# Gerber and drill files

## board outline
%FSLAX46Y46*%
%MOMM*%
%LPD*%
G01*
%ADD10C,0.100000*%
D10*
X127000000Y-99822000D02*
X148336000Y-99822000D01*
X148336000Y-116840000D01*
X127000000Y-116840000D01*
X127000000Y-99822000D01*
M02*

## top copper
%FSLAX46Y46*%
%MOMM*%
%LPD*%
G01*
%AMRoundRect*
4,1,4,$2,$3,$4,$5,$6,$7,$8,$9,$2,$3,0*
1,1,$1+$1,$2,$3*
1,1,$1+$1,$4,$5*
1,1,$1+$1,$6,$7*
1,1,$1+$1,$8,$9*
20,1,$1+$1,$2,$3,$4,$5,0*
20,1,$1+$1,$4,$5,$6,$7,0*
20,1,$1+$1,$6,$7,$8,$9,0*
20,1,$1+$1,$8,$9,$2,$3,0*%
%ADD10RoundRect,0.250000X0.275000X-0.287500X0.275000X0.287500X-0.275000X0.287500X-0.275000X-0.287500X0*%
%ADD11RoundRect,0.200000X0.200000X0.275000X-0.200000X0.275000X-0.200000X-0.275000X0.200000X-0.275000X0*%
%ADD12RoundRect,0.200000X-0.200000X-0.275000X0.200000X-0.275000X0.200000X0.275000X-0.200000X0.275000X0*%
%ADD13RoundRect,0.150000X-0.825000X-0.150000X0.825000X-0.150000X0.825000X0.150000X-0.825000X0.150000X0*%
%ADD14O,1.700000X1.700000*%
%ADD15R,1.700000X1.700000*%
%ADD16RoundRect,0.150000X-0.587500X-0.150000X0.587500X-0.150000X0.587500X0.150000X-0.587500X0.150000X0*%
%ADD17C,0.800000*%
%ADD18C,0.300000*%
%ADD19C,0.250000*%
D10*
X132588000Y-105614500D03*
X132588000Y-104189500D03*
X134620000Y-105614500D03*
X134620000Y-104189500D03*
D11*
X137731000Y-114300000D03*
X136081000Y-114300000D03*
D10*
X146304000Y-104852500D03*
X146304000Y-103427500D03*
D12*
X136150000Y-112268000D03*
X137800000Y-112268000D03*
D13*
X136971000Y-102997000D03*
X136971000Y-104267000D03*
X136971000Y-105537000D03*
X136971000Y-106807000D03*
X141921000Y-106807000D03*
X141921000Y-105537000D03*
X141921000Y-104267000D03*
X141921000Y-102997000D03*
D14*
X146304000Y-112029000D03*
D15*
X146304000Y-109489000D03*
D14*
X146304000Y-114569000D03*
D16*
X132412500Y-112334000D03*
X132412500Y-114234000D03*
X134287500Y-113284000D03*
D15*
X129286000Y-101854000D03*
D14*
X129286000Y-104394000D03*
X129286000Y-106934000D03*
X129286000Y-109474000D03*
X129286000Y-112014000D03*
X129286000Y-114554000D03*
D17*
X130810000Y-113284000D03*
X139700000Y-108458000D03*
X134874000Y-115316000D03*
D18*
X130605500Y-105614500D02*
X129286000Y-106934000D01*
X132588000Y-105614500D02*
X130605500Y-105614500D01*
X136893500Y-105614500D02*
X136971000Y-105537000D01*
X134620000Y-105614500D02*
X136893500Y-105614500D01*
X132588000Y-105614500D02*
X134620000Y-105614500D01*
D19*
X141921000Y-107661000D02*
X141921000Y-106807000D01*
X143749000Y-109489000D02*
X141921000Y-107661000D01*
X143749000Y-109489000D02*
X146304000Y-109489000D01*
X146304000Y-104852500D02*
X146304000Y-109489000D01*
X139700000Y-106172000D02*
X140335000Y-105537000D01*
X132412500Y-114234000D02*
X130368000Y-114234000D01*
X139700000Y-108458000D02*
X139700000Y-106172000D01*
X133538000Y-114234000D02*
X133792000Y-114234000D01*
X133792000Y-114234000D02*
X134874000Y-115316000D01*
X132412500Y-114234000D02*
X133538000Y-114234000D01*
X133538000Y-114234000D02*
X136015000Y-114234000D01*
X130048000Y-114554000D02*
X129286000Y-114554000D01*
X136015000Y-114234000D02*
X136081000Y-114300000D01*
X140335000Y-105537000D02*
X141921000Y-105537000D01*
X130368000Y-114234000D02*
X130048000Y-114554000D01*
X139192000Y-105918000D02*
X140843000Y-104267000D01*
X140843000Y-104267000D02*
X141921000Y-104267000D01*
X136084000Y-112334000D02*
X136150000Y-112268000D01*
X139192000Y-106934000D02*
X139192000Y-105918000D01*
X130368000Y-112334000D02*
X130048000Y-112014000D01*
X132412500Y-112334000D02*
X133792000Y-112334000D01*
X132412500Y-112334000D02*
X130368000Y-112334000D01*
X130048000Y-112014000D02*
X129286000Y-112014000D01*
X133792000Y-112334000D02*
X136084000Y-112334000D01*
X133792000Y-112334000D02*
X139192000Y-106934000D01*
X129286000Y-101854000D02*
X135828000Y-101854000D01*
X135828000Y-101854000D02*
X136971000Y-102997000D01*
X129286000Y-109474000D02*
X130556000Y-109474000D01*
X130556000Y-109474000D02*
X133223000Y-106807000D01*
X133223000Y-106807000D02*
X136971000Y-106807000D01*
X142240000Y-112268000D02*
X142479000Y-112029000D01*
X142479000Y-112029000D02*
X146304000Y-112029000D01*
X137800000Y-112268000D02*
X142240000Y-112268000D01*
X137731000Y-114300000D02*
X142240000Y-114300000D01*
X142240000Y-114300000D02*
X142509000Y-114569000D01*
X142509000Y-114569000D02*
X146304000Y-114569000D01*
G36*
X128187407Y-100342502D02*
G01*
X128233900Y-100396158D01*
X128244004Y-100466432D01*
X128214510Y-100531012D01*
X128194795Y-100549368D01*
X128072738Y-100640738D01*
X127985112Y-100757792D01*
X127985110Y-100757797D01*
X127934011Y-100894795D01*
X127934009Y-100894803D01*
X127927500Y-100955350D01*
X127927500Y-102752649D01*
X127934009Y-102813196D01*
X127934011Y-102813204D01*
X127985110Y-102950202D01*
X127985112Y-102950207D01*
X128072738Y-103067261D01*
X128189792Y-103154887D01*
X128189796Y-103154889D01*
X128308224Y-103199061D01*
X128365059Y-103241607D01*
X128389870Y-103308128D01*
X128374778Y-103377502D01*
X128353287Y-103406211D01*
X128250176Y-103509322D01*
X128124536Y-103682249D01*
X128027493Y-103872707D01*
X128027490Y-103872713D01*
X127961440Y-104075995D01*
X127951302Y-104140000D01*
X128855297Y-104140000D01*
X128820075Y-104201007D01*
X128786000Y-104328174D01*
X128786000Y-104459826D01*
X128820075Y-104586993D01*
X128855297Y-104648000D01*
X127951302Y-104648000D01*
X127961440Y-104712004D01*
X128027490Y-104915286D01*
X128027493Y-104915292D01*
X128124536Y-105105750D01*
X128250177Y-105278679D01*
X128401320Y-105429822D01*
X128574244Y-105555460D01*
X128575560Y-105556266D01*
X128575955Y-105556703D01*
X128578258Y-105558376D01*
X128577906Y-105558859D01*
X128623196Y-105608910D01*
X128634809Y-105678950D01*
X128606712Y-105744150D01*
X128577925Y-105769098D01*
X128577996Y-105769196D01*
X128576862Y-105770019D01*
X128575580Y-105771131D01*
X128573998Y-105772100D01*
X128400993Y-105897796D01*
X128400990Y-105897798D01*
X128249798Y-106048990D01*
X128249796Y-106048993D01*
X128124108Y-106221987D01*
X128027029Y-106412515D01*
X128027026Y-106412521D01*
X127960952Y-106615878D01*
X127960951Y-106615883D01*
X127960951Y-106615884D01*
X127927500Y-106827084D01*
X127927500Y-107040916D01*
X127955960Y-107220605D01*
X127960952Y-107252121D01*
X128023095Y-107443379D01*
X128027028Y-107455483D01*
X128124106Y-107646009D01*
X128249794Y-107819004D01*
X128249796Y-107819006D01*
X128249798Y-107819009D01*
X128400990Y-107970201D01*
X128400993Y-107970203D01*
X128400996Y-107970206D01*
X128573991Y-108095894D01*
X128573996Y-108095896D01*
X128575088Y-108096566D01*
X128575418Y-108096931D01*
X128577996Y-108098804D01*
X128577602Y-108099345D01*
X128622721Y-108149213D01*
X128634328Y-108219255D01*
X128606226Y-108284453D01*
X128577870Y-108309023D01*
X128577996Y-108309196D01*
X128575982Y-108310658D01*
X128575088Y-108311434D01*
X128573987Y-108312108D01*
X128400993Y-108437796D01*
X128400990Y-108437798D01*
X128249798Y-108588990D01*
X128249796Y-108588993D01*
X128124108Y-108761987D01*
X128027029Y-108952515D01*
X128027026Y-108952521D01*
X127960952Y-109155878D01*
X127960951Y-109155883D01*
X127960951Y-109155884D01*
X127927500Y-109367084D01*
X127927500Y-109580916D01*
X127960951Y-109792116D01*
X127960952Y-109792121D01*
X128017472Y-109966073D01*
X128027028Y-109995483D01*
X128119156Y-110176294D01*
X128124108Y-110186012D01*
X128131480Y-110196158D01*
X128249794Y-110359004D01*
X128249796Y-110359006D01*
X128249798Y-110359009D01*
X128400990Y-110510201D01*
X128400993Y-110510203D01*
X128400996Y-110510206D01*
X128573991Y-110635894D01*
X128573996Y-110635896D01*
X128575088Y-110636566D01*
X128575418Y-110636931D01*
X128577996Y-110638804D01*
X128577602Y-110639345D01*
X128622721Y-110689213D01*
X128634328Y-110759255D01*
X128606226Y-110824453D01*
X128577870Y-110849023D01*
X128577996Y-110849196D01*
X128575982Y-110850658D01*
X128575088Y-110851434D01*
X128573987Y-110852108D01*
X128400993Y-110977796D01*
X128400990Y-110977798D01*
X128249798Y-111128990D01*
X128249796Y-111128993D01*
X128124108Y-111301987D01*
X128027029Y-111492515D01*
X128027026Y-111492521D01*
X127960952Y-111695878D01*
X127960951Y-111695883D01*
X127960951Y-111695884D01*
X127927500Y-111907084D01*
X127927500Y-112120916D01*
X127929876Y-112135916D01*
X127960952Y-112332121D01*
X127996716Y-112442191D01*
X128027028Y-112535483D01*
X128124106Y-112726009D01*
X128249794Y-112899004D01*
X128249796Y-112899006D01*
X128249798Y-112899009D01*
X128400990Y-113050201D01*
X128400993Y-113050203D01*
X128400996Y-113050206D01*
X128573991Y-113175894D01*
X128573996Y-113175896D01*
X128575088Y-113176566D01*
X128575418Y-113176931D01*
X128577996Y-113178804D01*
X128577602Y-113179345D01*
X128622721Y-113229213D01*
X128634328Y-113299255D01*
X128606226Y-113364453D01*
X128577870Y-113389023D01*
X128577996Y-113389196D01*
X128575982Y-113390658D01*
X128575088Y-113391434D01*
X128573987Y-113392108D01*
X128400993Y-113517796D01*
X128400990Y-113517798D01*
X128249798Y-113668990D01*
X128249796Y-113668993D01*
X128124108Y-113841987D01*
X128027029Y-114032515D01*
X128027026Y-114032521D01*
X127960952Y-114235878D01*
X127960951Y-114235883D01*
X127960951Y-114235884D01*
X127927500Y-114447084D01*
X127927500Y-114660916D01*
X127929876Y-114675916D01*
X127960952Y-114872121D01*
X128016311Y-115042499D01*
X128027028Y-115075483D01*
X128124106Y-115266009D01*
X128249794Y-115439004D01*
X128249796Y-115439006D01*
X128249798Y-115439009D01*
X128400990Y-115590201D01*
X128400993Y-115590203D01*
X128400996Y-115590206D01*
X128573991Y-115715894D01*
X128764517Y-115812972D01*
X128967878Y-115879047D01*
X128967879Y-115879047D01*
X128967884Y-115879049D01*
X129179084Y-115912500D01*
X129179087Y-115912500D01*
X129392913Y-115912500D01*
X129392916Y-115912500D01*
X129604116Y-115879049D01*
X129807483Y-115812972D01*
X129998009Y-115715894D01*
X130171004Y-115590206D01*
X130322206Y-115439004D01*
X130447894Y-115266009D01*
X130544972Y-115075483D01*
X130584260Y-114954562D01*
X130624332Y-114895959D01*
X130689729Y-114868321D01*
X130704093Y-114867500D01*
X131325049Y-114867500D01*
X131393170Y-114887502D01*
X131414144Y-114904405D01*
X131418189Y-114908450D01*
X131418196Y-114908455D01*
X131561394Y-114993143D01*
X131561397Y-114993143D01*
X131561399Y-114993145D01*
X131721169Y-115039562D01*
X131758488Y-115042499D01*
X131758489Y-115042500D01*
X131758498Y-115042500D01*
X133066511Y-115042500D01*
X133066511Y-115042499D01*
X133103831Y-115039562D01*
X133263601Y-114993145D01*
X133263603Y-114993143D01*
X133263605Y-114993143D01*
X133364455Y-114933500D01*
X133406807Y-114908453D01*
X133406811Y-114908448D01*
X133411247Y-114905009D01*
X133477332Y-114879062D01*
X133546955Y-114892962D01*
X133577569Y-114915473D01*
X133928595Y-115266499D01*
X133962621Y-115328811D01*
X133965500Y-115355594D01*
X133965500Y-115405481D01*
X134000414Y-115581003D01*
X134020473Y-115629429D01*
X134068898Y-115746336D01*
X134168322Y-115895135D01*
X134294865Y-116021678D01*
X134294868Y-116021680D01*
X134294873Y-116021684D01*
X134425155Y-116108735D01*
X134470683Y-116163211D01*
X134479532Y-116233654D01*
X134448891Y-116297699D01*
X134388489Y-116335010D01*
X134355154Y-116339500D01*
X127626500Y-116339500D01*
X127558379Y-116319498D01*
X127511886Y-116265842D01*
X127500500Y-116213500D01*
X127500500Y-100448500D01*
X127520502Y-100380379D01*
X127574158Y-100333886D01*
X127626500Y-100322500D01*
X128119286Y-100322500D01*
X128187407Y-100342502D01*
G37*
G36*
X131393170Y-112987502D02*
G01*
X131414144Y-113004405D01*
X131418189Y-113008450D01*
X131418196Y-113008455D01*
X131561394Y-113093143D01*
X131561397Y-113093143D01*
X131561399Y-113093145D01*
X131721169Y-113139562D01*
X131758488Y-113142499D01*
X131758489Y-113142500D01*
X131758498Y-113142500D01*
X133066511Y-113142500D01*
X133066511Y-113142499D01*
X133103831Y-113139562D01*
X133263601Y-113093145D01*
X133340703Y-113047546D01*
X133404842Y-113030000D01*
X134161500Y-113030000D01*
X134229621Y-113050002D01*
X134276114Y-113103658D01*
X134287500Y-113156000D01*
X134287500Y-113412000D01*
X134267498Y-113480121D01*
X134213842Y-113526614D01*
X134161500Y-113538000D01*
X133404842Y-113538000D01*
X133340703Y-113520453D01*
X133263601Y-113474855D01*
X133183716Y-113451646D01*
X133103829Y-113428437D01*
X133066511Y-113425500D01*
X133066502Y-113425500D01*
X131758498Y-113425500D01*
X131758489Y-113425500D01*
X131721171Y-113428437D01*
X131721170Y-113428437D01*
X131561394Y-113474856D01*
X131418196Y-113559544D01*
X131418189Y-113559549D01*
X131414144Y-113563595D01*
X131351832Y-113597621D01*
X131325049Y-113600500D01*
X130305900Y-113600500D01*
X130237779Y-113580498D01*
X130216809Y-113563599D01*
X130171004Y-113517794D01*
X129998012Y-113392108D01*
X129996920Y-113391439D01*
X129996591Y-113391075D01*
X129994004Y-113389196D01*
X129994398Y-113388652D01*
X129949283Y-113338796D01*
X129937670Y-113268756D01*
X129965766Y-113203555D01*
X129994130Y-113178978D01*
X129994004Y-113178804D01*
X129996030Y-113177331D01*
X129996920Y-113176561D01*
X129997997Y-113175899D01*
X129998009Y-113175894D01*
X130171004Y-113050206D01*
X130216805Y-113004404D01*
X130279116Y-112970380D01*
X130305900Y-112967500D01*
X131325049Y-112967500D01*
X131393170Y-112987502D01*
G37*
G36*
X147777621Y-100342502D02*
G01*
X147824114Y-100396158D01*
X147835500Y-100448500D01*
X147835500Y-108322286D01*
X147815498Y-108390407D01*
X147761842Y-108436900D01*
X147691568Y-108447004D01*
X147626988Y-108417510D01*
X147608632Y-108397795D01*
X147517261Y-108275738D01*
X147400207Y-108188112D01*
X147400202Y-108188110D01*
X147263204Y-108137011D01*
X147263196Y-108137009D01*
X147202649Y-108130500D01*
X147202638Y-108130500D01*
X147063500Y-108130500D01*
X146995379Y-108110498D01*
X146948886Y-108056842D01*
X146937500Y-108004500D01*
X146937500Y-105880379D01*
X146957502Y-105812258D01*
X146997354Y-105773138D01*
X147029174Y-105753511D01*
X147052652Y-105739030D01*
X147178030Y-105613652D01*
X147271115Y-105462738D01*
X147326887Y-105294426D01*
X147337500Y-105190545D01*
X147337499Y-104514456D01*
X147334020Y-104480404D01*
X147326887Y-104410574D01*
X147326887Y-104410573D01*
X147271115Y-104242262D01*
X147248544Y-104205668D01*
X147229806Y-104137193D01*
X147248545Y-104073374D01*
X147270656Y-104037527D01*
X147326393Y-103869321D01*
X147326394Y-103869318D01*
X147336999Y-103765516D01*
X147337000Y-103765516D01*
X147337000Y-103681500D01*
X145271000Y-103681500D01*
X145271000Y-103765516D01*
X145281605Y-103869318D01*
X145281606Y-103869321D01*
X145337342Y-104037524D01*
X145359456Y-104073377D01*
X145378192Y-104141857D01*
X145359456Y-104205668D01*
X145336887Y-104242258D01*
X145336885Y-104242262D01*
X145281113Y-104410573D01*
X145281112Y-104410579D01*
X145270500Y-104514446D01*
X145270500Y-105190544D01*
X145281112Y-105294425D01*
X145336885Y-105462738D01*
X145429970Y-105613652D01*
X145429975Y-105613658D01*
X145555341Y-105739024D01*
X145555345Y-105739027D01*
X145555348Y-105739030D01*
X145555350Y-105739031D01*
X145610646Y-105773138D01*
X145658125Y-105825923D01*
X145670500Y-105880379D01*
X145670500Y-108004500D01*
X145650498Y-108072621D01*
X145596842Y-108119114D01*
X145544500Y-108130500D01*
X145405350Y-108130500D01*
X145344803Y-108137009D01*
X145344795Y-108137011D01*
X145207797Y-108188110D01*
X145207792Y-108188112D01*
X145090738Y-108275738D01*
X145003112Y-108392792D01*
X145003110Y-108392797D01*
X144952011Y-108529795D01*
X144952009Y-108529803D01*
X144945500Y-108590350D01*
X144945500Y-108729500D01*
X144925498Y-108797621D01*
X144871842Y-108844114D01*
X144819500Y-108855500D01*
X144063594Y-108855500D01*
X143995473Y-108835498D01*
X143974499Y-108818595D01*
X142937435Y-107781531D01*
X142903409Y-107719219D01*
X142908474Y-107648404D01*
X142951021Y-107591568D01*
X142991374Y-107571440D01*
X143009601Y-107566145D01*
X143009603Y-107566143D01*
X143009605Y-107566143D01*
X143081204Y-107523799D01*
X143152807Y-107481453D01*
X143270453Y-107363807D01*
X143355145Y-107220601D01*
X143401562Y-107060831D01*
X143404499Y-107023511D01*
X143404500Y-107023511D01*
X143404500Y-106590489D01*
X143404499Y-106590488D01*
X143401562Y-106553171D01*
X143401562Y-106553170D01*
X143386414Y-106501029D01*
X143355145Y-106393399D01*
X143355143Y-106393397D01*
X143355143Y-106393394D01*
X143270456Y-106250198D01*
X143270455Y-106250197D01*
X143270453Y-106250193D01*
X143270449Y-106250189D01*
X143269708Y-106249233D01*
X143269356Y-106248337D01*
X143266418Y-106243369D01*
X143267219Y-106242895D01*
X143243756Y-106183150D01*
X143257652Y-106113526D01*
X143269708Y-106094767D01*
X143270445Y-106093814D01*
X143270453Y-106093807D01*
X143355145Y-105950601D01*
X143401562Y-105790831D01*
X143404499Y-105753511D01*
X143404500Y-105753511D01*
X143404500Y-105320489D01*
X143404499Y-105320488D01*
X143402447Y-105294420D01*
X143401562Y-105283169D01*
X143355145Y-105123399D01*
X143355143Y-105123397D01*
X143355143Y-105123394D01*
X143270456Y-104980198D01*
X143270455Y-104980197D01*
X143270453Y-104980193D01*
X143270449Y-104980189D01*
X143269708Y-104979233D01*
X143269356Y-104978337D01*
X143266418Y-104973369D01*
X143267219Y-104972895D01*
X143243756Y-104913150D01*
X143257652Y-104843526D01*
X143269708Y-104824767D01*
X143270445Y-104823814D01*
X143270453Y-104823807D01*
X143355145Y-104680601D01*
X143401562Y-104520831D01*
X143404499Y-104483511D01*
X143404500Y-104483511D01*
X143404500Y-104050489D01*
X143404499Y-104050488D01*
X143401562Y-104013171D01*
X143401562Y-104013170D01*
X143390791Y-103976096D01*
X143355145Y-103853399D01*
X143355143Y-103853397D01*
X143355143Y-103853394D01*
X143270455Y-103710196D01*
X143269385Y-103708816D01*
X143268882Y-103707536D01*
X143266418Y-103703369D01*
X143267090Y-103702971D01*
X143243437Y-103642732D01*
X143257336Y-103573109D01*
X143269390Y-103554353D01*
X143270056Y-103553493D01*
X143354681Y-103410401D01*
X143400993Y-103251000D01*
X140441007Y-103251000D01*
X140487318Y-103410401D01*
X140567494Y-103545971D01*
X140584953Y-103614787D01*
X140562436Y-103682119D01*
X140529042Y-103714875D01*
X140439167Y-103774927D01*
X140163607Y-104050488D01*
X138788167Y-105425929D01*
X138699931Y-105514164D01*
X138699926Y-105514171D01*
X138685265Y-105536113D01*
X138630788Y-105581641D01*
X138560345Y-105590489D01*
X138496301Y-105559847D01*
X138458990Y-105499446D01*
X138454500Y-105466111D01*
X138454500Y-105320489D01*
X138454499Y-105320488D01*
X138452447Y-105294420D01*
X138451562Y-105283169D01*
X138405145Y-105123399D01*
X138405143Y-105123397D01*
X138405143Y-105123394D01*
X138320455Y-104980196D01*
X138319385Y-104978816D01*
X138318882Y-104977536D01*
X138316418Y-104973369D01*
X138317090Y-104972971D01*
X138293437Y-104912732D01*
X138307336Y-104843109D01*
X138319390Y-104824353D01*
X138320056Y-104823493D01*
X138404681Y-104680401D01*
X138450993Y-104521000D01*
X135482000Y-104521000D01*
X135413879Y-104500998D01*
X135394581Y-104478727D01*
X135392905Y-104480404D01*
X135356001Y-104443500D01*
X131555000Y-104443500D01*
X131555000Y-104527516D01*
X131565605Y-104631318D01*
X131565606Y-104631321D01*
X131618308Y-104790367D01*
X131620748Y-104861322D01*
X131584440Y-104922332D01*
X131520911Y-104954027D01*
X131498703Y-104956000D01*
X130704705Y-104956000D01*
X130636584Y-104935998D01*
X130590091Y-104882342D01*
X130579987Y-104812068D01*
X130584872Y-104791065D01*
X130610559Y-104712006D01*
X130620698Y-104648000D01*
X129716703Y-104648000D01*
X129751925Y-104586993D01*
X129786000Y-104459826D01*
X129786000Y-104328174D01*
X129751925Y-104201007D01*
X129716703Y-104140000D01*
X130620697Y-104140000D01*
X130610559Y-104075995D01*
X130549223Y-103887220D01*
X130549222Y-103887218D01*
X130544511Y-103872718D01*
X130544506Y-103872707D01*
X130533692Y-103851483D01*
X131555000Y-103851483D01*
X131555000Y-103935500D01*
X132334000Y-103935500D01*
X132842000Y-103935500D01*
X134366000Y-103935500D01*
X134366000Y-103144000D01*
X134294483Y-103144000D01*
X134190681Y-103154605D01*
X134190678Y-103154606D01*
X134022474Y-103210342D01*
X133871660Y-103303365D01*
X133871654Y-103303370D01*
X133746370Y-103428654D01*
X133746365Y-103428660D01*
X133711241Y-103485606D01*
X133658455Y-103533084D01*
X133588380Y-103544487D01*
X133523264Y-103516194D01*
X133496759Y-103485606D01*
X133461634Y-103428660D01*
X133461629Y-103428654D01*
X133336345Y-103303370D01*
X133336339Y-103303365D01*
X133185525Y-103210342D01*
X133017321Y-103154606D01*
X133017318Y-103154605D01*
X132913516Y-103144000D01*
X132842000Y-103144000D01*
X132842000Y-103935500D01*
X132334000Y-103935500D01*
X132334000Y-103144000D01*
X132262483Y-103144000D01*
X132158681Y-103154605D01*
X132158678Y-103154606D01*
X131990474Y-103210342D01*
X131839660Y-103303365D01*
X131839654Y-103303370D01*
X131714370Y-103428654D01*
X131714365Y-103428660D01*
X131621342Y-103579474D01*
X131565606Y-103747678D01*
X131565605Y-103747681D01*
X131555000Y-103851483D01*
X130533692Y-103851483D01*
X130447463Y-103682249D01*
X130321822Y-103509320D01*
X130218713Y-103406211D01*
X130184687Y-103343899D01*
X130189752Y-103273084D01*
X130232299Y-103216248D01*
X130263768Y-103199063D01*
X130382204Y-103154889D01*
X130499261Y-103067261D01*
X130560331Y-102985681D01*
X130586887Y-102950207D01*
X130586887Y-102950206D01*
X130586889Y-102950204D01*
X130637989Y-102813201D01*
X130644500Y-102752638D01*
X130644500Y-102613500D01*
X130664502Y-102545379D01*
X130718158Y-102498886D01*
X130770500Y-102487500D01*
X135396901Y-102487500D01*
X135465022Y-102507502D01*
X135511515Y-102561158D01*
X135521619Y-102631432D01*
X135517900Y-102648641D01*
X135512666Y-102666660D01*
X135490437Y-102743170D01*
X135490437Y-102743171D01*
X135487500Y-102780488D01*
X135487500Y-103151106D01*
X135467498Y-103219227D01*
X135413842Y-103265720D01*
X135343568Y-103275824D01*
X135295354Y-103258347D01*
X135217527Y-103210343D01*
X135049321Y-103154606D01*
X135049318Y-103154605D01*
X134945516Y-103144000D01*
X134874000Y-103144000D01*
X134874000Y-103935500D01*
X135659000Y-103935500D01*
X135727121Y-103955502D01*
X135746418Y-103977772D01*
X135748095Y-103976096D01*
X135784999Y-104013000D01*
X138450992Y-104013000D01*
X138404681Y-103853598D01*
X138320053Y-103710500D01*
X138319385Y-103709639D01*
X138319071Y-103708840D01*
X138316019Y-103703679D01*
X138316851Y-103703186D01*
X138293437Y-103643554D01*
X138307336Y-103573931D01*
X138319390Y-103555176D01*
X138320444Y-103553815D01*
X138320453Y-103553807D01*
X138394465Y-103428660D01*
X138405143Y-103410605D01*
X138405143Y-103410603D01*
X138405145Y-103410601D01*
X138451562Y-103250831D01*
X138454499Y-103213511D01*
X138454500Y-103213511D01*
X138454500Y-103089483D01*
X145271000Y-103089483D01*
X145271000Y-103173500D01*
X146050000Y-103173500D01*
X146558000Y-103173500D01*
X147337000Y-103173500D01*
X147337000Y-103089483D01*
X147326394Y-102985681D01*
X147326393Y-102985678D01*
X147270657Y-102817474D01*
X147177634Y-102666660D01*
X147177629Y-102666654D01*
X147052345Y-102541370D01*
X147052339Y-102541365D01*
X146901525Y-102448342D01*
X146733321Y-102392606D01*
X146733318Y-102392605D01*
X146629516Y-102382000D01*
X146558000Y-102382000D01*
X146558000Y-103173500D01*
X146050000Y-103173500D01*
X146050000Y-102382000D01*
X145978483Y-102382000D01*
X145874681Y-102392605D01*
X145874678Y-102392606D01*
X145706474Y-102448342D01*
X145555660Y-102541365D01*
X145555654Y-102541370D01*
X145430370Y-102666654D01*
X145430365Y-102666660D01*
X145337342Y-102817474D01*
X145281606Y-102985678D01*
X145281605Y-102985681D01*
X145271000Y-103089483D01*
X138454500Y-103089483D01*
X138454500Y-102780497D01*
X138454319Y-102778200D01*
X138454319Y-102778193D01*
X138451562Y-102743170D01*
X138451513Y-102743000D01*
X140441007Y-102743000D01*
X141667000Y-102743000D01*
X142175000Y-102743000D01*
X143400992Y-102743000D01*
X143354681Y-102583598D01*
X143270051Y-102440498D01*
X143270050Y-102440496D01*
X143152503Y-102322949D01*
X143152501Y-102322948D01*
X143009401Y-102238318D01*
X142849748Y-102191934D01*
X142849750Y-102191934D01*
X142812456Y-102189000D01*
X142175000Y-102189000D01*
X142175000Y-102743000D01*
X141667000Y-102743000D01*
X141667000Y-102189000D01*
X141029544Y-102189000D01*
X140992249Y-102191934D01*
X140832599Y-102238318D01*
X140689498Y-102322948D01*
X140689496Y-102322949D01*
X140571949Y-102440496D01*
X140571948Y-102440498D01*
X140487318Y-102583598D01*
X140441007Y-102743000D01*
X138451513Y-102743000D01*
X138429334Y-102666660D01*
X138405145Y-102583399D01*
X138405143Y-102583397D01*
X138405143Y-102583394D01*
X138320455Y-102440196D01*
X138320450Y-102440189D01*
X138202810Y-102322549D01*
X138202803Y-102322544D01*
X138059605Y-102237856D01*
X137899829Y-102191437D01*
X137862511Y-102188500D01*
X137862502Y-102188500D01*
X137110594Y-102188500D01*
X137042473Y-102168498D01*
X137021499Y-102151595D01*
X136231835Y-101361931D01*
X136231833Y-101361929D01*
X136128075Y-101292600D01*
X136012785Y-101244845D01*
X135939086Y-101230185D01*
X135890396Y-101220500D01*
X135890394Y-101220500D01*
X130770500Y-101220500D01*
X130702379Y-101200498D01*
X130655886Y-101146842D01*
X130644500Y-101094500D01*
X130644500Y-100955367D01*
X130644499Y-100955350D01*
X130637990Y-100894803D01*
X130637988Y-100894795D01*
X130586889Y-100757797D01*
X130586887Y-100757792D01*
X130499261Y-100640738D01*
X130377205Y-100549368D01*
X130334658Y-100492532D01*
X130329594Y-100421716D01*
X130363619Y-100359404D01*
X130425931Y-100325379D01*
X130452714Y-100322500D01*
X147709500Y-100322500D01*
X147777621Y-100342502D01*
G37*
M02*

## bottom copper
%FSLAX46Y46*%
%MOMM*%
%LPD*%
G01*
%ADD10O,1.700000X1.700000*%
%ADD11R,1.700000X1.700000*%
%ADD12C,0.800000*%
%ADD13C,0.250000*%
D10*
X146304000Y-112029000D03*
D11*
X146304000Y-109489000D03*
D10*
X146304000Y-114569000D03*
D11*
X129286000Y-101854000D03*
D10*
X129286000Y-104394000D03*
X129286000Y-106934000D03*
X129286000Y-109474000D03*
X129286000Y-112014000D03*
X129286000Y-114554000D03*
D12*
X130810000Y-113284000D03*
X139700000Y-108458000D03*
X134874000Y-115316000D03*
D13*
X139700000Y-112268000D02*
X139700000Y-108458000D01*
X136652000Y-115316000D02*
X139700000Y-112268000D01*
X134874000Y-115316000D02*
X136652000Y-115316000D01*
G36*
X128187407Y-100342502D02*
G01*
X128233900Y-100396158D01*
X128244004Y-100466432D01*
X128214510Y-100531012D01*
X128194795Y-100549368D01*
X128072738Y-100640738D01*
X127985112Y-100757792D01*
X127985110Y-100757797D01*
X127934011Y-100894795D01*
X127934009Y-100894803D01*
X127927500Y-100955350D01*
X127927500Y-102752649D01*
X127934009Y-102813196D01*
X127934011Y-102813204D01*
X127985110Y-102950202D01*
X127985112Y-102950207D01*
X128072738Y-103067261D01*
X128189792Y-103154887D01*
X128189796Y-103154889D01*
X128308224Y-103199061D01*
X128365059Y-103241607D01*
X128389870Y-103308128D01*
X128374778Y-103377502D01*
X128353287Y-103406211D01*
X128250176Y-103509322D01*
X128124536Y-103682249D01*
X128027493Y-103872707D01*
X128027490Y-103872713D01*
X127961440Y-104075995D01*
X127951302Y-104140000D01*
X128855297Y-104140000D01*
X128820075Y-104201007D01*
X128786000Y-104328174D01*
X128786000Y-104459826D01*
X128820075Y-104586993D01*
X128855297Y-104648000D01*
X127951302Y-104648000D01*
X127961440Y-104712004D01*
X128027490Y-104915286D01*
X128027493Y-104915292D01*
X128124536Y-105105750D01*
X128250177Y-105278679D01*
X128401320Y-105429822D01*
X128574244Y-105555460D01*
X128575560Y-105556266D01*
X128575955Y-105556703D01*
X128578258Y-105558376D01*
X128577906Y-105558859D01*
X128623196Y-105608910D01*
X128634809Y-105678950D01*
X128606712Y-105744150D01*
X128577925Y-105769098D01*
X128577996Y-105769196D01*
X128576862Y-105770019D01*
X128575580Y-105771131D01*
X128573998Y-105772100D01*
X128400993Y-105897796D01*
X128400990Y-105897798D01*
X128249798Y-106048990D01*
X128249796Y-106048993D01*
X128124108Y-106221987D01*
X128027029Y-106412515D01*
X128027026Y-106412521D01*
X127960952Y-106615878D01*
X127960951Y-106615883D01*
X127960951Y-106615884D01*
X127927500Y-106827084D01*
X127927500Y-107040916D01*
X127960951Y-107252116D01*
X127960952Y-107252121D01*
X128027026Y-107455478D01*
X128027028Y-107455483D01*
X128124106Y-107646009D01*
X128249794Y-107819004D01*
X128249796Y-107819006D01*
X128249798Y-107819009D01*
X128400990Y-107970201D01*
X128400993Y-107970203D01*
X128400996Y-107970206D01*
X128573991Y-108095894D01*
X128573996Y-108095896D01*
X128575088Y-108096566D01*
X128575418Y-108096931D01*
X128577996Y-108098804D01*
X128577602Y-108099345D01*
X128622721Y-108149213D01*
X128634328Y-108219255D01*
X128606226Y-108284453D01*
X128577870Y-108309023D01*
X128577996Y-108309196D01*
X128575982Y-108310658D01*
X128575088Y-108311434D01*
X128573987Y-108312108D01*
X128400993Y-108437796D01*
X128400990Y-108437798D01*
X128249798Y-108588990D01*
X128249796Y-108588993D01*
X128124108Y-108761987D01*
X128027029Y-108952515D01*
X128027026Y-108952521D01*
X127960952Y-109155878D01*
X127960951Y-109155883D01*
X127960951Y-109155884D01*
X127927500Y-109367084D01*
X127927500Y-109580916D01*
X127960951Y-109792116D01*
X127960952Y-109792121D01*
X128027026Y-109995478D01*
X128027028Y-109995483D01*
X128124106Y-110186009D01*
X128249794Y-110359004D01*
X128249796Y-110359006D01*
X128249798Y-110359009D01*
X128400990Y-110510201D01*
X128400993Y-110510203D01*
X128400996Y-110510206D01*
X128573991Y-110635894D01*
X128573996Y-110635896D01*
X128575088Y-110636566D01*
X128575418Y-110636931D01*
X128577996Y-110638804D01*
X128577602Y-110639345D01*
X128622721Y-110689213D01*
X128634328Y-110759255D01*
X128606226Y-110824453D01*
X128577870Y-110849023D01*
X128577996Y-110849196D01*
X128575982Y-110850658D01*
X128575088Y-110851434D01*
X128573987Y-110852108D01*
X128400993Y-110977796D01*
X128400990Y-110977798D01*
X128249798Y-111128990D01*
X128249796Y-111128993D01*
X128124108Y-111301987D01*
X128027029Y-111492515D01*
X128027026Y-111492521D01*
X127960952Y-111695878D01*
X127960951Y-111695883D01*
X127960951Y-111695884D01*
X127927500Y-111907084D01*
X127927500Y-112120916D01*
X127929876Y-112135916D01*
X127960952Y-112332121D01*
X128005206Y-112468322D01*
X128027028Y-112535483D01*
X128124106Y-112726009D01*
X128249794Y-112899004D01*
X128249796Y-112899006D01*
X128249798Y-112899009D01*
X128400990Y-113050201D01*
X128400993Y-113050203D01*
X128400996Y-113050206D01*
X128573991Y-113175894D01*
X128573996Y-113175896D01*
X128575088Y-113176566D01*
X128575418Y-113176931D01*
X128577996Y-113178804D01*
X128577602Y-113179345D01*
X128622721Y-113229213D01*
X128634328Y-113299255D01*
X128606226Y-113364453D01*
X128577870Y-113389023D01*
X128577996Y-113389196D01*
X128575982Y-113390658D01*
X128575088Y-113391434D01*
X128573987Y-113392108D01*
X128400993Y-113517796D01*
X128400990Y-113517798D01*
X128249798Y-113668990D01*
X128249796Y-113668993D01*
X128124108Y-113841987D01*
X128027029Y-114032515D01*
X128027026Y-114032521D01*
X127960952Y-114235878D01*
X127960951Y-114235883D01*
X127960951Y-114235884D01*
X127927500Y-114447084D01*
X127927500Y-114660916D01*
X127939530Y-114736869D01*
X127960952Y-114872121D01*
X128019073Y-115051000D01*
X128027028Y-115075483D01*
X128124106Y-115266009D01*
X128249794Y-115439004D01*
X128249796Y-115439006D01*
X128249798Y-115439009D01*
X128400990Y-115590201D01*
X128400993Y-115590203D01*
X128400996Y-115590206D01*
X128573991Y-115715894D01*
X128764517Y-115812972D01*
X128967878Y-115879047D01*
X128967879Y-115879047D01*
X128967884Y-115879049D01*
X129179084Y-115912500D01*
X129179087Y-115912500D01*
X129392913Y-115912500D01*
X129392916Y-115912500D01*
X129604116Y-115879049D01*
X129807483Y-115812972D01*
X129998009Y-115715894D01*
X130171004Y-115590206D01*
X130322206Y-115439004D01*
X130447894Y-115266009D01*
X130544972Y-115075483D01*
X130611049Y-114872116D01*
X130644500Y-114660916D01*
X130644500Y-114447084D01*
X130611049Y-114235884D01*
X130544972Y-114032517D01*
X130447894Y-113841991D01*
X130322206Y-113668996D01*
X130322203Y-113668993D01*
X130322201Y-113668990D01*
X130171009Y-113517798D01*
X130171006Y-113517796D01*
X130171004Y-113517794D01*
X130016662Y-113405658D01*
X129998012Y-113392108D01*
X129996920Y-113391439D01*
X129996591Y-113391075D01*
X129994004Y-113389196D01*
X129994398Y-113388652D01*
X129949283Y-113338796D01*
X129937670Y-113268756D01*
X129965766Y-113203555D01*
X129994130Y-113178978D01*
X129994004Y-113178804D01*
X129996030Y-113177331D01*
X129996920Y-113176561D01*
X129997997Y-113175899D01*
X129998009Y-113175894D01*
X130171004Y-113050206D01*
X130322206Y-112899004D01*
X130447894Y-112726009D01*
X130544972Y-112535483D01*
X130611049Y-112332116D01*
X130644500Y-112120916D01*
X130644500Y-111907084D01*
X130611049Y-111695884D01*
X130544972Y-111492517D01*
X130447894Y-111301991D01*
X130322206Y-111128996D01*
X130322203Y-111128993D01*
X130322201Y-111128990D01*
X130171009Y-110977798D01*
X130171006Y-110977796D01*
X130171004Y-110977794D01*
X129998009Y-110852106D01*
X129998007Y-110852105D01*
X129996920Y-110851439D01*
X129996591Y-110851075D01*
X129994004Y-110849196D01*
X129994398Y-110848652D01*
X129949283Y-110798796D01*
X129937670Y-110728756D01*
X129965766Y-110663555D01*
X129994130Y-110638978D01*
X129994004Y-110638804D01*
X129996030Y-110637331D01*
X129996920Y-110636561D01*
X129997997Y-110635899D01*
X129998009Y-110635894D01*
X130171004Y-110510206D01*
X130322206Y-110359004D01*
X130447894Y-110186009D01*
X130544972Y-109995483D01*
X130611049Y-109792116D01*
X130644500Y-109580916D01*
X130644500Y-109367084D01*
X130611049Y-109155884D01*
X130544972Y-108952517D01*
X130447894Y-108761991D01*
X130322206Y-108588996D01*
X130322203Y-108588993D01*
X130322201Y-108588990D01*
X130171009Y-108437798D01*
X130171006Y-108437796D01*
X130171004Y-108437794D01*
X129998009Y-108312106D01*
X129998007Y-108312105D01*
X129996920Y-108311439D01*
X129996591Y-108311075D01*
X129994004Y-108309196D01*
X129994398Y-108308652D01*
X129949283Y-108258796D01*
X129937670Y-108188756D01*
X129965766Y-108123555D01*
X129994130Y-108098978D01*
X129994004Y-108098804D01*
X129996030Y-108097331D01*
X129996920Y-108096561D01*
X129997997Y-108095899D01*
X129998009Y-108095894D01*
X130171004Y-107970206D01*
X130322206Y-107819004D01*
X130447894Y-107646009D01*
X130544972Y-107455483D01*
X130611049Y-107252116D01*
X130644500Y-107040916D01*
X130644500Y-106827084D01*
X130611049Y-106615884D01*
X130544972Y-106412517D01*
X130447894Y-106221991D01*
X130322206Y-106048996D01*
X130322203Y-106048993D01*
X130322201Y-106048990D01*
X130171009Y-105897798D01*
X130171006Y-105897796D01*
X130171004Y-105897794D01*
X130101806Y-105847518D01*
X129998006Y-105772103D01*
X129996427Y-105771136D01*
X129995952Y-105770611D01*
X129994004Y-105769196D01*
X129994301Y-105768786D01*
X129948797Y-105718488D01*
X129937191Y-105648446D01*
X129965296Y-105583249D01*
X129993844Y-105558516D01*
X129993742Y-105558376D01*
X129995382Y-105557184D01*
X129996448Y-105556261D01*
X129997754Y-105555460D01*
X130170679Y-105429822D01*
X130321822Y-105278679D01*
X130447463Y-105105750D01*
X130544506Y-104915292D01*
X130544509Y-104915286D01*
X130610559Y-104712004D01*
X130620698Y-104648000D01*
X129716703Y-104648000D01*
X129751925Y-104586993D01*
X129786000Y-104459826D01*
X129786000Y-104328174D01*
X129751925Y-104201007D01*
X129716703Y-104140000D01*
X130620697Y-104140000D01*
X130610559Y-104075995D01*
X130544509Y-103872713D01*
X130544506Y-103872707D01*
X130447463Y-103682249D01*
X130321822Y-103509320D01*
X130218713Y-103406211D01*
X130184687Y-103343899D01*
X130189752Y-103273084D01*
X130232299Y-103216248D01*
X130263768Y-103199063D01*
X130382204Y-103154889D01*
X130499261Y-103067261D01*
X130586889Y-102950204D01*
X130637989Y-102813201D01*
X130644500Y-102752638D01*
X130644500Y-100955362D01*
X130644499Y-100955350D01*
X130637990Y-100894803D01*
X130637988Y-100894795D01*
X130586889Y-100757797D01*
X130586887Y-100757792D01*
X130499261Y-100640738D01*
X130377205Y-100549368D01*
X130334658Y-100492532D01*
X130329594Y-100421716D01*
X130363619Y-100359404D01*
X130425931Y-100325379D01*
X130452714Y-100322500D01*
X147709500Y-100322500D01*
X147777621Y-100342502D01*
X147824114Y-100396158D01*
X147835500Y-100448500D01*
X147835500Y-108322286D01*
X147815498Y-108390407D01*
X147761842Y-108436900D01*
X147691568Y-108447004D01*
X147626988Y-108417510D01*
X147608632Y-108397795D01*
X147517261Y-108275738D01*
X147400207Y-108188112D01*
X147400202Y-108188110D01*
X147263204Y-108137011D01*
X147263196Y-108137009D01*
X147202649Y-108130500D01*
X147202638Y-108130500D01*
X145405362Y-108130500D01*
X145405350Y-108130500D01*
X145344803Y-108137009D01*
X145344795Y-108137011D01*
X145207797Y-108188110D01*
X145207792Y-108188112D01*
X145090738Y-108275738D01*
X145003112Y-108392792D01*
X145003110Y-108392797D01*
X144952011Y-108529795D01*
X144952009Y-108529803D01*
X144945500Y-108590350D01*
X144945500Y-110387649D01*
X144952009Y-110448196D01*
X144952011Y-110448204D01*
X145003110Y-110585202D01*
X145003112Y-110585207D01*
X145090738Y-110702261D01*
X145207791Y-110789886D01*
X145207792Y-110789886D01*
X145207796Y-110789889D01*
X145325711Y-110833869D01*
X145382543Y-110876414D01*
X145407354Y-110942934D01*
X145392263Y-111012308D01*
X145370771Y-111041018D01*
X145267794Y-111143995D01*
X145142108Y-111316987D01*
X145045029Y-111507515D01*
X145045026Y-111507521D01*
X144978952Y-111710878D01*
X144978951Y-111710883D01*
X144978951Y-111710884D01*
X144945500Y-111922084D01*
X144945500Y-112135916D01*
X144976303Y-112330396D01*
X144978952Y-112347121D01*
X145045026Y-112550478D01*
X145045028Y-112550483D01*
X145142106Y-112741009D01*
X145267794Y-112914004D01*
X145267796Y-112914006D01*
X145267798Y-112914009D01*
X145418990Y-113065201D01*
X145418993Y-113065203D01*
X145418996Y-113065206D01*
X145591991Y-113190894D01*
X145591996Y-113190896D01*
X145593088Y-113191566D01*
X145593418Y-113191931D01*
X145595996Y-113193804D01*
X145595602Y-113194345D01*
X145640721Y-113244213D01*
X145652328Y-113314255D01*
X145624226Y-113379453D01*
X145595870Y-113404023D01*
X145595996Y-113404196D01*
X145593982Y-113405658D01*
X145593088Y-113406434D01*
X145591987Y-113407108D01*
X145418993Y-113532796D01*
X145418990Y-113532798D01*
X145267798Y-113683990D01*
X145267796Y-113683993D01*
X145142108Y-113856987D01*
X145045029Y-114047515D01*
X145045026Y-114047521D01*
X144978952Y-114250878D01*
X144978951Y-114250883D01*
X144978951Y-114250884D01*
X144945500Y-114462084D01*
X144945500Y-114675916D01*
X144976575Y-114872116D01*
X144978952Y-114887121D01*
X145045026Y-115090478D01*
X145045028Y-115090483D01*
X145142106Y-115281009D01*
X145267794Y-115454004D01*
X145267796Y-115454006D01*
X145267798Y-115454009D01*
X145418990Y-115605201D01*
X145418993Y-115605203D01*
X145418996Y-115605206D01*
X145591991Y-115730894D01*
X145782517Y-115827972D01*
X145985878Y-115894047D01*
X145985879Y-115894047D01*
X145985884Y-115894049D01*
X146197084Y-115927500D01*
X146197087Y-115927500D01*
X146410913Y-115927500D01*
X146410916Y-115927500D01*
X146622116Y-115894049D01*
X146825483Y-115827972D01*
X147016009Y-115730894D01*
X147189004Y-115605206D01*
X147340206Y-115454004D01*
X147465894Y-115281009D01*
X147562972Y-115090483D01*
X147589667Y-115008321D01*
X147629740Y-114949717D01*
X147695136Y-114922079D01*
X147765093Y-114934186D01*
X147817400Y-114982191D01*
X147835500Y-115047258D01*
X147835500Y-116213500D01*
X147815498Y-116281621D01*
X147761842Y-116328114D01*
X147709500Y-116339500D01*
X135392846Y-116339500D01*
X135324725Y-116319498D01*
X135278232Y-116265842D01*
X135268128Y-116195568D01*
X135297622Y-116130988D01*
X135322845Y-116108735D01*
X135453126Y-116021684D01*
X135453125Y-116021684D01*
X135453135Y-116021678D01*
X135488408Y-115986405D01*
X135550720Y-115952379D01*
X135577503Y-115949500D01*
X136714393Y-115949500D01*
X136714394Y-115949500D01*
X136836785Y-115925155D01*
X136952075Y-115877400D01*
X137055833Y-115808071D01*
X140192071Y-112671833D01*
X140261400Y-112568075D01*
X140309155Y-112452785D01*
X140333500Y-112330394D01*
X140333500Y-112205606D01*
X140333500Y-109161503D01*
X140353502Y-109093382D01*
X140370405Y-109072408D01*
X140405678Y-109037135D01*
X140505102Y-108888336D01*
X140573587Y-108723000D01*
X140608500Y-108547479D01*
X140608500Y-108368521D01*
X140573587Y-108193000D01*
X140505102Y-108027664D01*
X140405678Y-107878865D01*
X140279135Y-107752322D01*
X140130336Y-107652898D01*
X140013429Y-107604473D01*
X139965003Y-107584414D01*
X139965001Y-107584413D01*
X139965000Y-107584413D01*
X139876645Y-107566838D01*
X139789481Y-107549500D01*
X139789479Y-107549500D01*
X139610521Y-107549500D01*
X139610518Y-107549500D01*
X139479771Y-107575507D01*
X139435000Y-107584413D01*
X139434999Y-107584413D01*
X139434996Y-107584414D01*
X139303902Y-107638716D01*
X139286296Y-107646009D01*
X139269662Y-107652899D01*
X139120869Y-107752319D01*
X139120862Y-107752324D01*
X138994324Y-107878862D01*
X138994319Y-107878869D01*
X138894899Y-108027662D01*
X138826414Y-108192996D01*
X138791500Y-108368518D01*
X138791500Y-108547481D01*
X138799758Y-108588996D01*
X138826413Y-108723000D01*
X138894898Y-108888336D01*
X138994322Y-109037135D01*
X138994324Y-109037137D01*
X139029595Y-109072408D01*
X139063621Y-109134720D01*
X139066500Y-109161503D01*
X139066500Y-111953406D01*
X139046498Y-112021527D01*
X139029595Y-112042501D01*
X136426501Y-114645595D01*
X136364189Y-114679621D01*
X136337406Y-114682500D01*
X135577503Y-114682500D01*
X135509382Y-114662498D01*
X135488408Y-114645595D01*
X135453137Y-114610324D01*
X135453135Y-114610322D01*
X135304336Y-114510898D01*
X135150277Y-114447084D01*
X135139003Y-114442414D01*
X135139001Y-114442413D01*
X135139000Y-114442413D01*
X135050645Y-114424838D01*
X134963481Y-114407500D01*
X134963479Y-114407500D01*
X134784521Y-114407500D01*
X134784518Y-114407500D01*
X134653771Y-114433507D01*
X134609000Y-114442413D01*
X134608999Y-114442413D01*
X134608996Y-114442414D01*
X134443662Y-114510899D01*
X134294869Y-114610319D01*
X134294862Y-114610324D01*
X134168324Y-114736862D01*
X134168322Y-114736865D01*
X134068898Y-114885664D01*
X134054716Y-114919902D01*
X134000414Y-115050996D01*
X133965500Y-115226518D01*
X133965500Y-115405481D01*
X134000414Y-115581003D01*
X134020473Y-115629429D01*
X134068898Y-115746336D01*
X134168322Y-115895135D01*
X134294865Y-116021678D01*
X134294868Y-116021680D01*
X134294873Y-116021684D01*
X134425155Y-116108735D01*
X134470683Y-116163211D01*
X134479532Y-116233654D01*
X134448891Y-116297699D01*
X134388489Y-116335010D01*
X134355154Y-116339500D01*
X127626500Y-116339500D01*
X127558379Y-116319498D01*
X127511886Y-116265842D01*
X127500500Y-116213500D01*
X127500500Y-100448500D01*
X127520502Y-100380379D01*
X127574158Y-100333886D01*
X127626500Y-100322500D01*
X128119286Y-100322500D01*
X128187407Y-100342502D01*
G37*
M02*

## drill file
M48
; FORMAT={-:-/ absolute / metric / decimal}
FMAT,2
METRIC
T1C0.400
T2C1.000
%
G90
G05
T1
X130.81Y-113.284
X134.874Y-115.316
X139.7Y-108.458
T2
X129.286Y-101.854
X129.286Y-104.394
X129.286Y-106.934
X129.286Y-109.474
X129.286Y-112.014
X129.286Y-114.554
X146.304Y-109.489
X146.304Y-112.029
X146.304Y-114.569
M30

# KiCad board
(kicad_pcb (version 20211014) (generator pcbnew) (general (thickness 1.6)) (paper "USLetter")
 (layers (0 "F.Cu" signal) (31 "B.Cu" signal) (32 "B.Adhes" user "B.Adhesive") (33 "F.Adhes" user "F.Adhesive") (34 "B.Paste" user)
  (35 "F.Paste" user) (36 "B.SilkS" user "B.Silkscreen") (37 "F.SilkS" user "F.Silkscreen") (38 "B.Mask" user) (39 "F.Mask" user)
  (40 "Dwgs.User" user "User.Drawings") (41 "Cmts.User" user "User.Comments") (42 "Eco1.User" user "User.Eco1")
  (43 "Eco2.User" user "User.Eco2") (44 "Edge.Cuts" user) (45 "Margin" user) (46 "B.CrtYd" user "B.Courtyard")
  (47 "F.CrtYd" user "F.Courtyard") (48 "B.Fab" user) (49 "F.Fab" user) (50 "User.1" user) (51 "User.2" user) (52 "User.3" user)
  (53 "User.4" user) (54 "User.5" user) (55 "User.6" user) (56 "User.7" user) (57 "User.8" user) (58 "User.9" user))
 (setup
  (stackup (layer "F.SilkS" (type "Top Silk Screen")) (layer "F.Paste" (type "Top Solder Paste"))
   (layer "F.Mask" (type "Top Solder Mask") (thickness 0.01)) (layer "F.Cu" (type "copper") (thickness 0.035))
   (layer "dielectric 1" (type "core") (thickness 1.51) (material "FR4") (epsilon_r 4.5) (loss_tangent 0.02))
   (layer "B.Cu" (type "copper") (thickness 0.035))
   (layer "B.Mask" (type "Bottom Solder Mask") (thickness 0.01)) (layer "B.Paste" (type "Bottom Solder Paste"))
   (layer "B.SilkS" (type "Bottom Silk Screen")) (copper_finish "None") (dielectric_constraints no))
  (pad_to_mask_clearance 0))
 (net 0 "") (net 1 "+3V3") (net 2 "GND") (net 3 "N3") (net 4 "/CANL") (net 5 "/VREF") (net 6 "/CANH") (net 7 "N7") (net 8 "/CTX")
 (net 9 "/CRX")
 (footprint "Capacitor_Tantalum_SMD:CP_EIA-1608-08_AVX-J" (layer "F.Cu") (at 132.588 104.902 90)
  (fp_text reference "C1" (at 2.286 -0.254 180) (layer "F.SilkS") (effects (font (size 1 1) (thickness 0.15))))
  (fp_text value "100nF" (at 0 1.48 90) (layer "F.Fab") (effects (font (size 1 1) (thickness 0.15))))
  (pad "1" smd roundrect (at -0.7125 0 90) (size 1.075 1.05) (layers "F.Cu" "F.Paste" "F.Mask") (roundrect_rratio 0.238095) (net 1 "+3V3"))
  (pad "2" smd roundrect (at 0.7125 0 90) (size 1.075 1.05) (layers "F.Cu" "F.Paste" "F.Mask") (roundrect_rratio 0.238095) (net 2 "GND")))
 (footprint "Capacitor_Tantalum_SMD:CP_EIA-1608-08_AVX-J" (layer "F.Cu") (at 134.62 104.902 90)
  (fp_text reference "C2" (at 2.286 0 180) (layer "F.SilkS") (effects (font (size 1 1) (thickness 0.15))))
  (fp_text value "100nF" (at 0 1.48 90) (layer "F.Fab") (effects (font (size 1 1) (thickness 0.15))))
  (pad "1" smd roundrect (at -0.7125 0 90) (size 1.075 1.05) (layers "F.Cu" "F.Paste" "F.Mask") (roundrect_rratio 0.238095) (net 1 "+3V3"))
  (pad "2" smd roundrect (at 0.7125 0 90) (size 1.075 1.05) (layers "F.Cu" "F.Paste" "F.Mask") (roundrect_rratio 0.238095) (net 2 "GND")))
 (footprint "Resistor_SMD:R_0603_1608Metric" (layer "F.Cu") (at 136.906 114.3 180)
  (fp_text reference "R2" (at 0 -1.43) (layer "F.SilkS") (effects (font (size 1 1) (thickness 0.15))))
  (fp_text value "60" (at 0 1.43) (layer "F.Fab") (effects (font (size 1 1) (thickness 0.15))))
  (pad "1" smd roundrect (at -0.825 0 180) (size 0.8 0.95) (layers "F.Cu" "F.Paste" "F.Mask") (roundrect_rratio 0.25) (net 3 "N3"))
  (pad "2" smd roundrect (at 0.825 0 180) (size 0.8 0.95) (layers "F.Cu" "F.Paste" "F.Mask") (roundrect_rratio 0.25) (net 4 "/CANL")))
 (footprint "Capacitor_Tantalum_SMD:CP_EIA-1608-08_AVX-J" (layer "F.Cu") (at 146.304 104.14 90)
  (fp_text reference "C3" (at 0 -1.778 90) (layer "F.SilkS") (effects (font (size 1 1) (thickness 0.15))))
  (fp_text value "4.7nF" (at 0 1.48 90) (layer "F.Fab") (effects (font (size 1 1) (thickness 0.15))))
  (pad "1" smd roundrect (at -0.7125 0 90) (size 1.075 1.05) (layers "F.Cu" "F.Paste" "F.Mask") (roundrect_rratio 0.238095) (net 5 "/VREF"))
  (pad "2" smd roundrect (at 0.7125 0 90) (size 1.075 1.05) (layers "F.Cu" "F.Paste" "F.Mask") (roundrect_rratio 0.238095) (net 2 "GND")))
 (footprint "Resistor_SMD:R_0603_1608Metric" (layer "F.Cu") (at 136.975 112.268)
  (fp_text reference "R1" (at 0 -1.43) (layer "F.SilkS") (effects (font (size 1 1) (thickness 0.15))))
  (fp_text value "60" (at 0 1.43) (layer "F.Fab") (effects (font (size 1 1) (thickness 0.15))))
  (pad "1" smd roundrect (at -0.825 0) (size 0.8 0.95) (layers "F.Cu" "F.Paste" "F.Mask") (roundrect_rratio 0.25) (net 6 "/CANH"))
  (pad "2" smd roundrect (at 0.825 0) (size 0.8 0.95) (layers "F.Cu" "F.Paste" "F.Mask") (roundrect_rratio 0.25) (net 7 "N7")))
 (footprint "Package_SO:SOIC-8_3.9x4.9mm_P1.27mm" (layer "F.Cu") (at 139.446 104.902)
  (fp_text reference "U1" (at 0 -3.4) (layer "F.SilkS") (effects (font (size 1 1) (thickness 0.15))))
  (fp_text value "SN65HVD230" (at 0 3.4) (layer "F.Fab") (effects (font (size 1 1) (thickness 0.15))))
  (pad "1" smd roundrect (at -2.475 -1.905) (size 1.95 0.6) (layers "F.Cu" "F.Paste" "F.Mask") (roundrect_rratio 0.25) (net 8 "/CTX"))
  (pad "2" smd roundrect (at -2.475 -0.635) (size 1.95 0.6) (layers "F.Cu" "F.Paste" "F.Mask") (roundrect_rratio 0.25) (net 2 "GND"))
  (pad "3" smd roundrect (at -2.475 0.635) (size 1.95 0.6) (layers "F.Cu" "F.Paste" "F.Mask") (roundrect_rratio 0.25) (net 1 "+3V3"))
  (pad "4" smd roundrect (at -2.475 1.905) (size 1.95 0.6) (layers "F.Cu" "F.Paste" "F.Mask") (roundrect_rratio 0.25) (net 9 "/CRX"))
  (pad "5" smd roundrect (at 2.475 1.905) (size 1.95 0.6) (layers "F.Cu" "F.Paste" "F.Mask") (roundrect_rratio 0.25) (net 5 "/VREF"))
  (pad "6" smd roundrect (at 2.475 0.635) (size 1.95 0.6) (layers "F.Cu" "F.Paste" "F.Mask") (roundrect_rratio 0.25) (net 4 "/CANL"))
  (pad "7" smd roundrect (at 2.475 -0.635) (size 1.95 0.6) (layers "F.Cu" "F.Paste" "F.Mask") (roundrect_rratio 0.25) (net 6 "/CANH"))
  (pad "8" smd roundrect (at 2.475 -1.905) (size 1.95 0.6) (layers "F.Cu" "F.Paste" "F.Mask") (roundrect_rratio 0.25) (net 2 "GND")))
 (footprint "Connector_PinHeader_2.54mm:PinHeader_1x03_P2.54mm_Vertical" (layer "F.Cu") (at 146.304 109.489)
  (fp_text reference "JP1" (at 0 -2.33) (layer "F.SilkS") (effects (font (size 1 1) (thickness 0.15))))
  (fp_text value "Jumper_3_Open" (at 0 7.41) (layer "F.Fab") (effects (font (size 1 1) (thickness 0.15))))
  (pad "1" thru_hole oval (at 0 2.54) (size 1.7 1.7) (drill 1) (layers *.Cu *.Mask) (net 7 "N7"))
  (pad "2" thru_hole rect (at 0 0) (size 1.7 1.7) (drill 1) (layers *.Cu *.Mask) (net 5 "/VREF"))
  (pad "3" thru_hole oval (at 0 5.08) (size 1.7 1.7) (drill 1) (layers *.Cu *.Mask) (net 3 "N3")))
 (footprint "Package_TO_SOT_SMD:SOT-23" (layer "F.Cu") (at 133.35 113.284)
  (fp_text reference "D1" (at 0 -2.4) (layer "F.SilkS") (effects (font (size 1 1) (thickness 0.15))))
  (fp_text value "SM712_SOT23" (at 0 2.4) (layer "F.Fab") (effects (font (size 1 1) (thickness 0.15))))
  (pad "1" smd roundrect (at -0.9375 -0.95) (size 1.475 0.6) (layers "F.Cu" "F.Paste" "F.Mask") (roundrect_rratio 0.25) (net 6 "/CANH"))
  (pad "2" smd roundrect (at -0.9375 0.95) (size 1.475 0.6) (layers "F.Cu" "F.Paste" "F.Mask") (roundrect_rratio 0.25) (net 4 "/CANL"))
  (pad "3" smd roundrect (at 0.9375 0) (size 1.475 0.6) (layers "F.Cu" "F.Paste" "F.Mask") (roundrect_rratio 0.25) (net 2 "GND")))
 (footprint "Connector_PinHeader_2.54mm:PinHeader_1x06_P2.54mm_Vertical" (layer "B.Cu") (at 129.286 101.854 180)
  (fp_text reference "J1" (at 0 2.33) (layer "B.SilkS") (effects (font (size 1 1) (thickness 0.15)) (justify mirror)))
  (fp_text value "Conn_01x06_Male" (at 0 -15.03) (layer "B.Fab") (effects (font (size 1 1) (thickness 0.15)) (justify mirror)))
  (pad "1" thru_hole rect (at 0 0 180) (size 1.7 1.7) (drill 1) (layers *.Cu *.Mask) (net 8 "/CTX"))
  (pad "2" thru_hole oval (at 0 -2.54 180) (size 1.7 1.7) (drill 1) (layers *.Cu *.Mask) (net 2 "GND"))
  (pad "3" thru_hole oval (at 0 -5.08 180) (size 1.7 1.7) (drill 1) (layers *.Cu *.Mask) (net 1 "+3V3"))
  (pad "4" thru_hole oval (at 0 -7.62 180) (size 1.7 1.7) (drill 1) (layers *.Cu *.Mask) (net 9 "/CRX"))
  (pad "5" thru_hole oval (at 0 -10.16 180) (size 1.7 1.7) (drill 1) (layers *.Cu *.Mask) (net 6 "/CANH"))
  (pad "6" thru_hole oval (at 0 -12.7 180) (size 1.7 1.7) (drill 1) (layers *.Cu *.Mask) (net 4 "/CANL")))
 (gr_rect (start 127 99.822) (end 148.336 116.84) (layer "Edge.Cuts") (width 0.1) (fill none))
 (segment (start 130.6055 105.6145) (end 129.286 106.934) (width 0.3) (layer "F.Cu") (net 1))
 (segment (start 132.588 105.6145) (end 130.6055 105.6145) (width 0.3) (layer "F.Cu") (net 1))
 (segment (start 136.8935 105.6145) (end 136.971 105.537) (width 0.3) (layer "F.Cu") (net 1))
 (segment (start 134.62 105.6145) (end 136.8935 105.6145) (width 0.3) (layer "F.Cu") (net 1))
 (segment (start 132.588 105.6145) (end 134.62 105.6145) (width 0.3) (layer "F.Cu") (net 1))
 (via (at 130.81 113.284) (size 0.8) (drill 0.4) (layers "F.Cu" "B.Cu") (free) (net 2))
 (segment (start 141.921 107.661) (end 141.921 106.807) (width 0.25) (layer "F.Cu") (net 5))
 (segment (start 143.749 109.489) (end 141.921 107.661) (width 0.25) (layer "F.Cu") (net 5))
 (segment (start 143.749 109.489) (end 146.304 109.489) (width 0.25) (layer "F.Cu") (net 5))
 (segment (start 146.304 104.8525) (end 146.304 109.489) (width 0.25) (layer "F.Cu") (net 5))
 (segment (start 139.7 106.172) (end 140.335 105.537) (width 0.25) (layer "F.Cu") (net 4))
 (segment (start 132.4125 114.234) (end 130.368 114.234) (width 0.25) (layer "F.Cu") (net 4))
 (segment (start 139.7 108.458) (end 139.7 106.172) (width 0.25) (layer "F.Cu") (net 4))
 (segment (start 133.538 114.234) (end 133.792 114.234) (width 0.25) (layer "F.Cu") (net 4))
 (segment (start 133.792 114.234) (end 134.874 115.316) (width 0.25) (layer "F.Cu") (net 4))
 (segment (start 132.4125 114.234) (end 133.538 114.234) (width 0.25) (layer "F.Cu") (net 4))
 (segment (start 133.538 114.234) (end 136.015 114.234) (width 0.25) (layer "F.Cu") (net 4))
 (segment (start 130.048 114.554) (end 129.286 114.554) (width 0.25) (layer "F.Cu") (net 4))
 (segment (start 136.015 114.234) (end 136.081 114.3) (width 0.25) (layer "F.Cu") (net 4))
 (segment (start 140.335 105.537) (end 141.921 105.537) (width 0.25) (layer "F.Cu") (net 4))
 (segment (start 130.368 114.234) (end 130.048 114.554) (width 0.25) (layer "F.Cu") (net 4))
 (via (at 139.7 108.458) (size 0.8) (drill 0.4) (layers "F.Cu" "B.Cu") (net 4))
 (via (at 134.874 115.316) (size 0.8) (drill 0.4) (layers "F.Cu" "B.Cu") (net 4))
 (segment (start 139.7 112.268) (end 139.7 108.458) (width 0.25) (layer "B.Cu") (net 4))
 (segment (start 136.652 115.316) (end 139.7 112.268) (width 0.25) (layer "B.Cu") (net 4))
 (segment (start 134.874 115.316) (end 136.652 115.316) (width 0.25) (layer "B.Cu") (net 4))
 (segment (start 139.192 105.918) (end 140.843 104.267) (width 0.25) (layer "F.Cu") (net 6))
 (segment (start 140.843 104.267) (end 141.921 104.267) (width 0.25) (layer "F.Cu") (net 6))
 (segment (start 136.084 112.334) (end 136.15 112.268) (width 0.25) (layer "F.Cu") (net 6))
 (segment (start 139.192 106.934) (end 139.192 105.918) (width 0.25) (layer "F.Cu") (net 6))
 (segment (start 130.368 112.334) (end 130.048 112.014) (width 0.25) (layer "F.Cu") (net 6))
 (segment (start 132.4125 112.334) (end 133.792 112.334) (width 0.25) (layer "F.Cu") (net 6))
 (segment (start 132.4125 112.334) (end 130.368 112.334) (width 0.25) (layer "F.Cu") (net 6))
 (segment (start 130.048 112.014) (end 129.286 112.014) (width 0.25) (layer "F.Cu") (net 6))
 (segment (start 133.792 112.334) (end 136.084 112.334) (width 0.25) (layer "F.Cu") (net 6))
 (segment (start 133.792 112.334) (end 139.192 106.934) (width 0.25) (layer "F.Cu") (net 6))
 (segment (start 129.286 101.854) (end 135.828 101.854) (width 0.25) (layer "F.Cu") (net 8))
 (segment (start 135.828 101.854) (end 136.971 102.997) (width 0.25) (layer "F.Cu") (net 8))
 (segment (start 129.286 109.474) (end 130.556 109.474) (width 0.25) (layer "F.Cu") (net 9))
 (segment (start 130.556 109.474) (end 133.223 106.807) (width 0.25) (layer "F.Cu") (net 9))
 (segment (start 133.223 106.807) (end 136.971 106.807) (width 0.25) (layer "F.Cu") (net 9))
 (segment (start 142.24 112.268) (end 142.479 112.029) (width 0.25) (layer "F.Cu") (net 7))
 (segment (start 142.479 112.029) (end 146.304 112.029) (width 0.25) (layer "F.Cu") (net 7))
 (segment (start 137.8 112.268) (end 142.24 112.268) (width 0.25) (layer "F.Cu") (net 7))
 (segment (start 137.731 114.3) (end 142.24 114.3) (width 0.25) (layer "F.Cu") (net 3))
 (segment (start 142.24 114.3) (end 142.509 114.569) (width 0.25) (layer "F.Cu") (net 3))
 (segment (start 142.509 114.569) (end 146.304 114.569) (width 0.25) (layer "F.Cu") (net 3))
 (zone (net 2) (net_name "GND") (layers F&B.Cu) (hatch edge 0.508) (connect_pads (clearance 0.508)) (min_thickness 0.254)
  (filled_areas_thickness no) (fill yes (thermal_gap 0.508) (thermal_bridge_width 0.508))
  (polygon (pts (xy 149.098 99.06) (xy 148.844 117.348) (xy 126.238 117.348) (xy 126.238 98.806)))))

